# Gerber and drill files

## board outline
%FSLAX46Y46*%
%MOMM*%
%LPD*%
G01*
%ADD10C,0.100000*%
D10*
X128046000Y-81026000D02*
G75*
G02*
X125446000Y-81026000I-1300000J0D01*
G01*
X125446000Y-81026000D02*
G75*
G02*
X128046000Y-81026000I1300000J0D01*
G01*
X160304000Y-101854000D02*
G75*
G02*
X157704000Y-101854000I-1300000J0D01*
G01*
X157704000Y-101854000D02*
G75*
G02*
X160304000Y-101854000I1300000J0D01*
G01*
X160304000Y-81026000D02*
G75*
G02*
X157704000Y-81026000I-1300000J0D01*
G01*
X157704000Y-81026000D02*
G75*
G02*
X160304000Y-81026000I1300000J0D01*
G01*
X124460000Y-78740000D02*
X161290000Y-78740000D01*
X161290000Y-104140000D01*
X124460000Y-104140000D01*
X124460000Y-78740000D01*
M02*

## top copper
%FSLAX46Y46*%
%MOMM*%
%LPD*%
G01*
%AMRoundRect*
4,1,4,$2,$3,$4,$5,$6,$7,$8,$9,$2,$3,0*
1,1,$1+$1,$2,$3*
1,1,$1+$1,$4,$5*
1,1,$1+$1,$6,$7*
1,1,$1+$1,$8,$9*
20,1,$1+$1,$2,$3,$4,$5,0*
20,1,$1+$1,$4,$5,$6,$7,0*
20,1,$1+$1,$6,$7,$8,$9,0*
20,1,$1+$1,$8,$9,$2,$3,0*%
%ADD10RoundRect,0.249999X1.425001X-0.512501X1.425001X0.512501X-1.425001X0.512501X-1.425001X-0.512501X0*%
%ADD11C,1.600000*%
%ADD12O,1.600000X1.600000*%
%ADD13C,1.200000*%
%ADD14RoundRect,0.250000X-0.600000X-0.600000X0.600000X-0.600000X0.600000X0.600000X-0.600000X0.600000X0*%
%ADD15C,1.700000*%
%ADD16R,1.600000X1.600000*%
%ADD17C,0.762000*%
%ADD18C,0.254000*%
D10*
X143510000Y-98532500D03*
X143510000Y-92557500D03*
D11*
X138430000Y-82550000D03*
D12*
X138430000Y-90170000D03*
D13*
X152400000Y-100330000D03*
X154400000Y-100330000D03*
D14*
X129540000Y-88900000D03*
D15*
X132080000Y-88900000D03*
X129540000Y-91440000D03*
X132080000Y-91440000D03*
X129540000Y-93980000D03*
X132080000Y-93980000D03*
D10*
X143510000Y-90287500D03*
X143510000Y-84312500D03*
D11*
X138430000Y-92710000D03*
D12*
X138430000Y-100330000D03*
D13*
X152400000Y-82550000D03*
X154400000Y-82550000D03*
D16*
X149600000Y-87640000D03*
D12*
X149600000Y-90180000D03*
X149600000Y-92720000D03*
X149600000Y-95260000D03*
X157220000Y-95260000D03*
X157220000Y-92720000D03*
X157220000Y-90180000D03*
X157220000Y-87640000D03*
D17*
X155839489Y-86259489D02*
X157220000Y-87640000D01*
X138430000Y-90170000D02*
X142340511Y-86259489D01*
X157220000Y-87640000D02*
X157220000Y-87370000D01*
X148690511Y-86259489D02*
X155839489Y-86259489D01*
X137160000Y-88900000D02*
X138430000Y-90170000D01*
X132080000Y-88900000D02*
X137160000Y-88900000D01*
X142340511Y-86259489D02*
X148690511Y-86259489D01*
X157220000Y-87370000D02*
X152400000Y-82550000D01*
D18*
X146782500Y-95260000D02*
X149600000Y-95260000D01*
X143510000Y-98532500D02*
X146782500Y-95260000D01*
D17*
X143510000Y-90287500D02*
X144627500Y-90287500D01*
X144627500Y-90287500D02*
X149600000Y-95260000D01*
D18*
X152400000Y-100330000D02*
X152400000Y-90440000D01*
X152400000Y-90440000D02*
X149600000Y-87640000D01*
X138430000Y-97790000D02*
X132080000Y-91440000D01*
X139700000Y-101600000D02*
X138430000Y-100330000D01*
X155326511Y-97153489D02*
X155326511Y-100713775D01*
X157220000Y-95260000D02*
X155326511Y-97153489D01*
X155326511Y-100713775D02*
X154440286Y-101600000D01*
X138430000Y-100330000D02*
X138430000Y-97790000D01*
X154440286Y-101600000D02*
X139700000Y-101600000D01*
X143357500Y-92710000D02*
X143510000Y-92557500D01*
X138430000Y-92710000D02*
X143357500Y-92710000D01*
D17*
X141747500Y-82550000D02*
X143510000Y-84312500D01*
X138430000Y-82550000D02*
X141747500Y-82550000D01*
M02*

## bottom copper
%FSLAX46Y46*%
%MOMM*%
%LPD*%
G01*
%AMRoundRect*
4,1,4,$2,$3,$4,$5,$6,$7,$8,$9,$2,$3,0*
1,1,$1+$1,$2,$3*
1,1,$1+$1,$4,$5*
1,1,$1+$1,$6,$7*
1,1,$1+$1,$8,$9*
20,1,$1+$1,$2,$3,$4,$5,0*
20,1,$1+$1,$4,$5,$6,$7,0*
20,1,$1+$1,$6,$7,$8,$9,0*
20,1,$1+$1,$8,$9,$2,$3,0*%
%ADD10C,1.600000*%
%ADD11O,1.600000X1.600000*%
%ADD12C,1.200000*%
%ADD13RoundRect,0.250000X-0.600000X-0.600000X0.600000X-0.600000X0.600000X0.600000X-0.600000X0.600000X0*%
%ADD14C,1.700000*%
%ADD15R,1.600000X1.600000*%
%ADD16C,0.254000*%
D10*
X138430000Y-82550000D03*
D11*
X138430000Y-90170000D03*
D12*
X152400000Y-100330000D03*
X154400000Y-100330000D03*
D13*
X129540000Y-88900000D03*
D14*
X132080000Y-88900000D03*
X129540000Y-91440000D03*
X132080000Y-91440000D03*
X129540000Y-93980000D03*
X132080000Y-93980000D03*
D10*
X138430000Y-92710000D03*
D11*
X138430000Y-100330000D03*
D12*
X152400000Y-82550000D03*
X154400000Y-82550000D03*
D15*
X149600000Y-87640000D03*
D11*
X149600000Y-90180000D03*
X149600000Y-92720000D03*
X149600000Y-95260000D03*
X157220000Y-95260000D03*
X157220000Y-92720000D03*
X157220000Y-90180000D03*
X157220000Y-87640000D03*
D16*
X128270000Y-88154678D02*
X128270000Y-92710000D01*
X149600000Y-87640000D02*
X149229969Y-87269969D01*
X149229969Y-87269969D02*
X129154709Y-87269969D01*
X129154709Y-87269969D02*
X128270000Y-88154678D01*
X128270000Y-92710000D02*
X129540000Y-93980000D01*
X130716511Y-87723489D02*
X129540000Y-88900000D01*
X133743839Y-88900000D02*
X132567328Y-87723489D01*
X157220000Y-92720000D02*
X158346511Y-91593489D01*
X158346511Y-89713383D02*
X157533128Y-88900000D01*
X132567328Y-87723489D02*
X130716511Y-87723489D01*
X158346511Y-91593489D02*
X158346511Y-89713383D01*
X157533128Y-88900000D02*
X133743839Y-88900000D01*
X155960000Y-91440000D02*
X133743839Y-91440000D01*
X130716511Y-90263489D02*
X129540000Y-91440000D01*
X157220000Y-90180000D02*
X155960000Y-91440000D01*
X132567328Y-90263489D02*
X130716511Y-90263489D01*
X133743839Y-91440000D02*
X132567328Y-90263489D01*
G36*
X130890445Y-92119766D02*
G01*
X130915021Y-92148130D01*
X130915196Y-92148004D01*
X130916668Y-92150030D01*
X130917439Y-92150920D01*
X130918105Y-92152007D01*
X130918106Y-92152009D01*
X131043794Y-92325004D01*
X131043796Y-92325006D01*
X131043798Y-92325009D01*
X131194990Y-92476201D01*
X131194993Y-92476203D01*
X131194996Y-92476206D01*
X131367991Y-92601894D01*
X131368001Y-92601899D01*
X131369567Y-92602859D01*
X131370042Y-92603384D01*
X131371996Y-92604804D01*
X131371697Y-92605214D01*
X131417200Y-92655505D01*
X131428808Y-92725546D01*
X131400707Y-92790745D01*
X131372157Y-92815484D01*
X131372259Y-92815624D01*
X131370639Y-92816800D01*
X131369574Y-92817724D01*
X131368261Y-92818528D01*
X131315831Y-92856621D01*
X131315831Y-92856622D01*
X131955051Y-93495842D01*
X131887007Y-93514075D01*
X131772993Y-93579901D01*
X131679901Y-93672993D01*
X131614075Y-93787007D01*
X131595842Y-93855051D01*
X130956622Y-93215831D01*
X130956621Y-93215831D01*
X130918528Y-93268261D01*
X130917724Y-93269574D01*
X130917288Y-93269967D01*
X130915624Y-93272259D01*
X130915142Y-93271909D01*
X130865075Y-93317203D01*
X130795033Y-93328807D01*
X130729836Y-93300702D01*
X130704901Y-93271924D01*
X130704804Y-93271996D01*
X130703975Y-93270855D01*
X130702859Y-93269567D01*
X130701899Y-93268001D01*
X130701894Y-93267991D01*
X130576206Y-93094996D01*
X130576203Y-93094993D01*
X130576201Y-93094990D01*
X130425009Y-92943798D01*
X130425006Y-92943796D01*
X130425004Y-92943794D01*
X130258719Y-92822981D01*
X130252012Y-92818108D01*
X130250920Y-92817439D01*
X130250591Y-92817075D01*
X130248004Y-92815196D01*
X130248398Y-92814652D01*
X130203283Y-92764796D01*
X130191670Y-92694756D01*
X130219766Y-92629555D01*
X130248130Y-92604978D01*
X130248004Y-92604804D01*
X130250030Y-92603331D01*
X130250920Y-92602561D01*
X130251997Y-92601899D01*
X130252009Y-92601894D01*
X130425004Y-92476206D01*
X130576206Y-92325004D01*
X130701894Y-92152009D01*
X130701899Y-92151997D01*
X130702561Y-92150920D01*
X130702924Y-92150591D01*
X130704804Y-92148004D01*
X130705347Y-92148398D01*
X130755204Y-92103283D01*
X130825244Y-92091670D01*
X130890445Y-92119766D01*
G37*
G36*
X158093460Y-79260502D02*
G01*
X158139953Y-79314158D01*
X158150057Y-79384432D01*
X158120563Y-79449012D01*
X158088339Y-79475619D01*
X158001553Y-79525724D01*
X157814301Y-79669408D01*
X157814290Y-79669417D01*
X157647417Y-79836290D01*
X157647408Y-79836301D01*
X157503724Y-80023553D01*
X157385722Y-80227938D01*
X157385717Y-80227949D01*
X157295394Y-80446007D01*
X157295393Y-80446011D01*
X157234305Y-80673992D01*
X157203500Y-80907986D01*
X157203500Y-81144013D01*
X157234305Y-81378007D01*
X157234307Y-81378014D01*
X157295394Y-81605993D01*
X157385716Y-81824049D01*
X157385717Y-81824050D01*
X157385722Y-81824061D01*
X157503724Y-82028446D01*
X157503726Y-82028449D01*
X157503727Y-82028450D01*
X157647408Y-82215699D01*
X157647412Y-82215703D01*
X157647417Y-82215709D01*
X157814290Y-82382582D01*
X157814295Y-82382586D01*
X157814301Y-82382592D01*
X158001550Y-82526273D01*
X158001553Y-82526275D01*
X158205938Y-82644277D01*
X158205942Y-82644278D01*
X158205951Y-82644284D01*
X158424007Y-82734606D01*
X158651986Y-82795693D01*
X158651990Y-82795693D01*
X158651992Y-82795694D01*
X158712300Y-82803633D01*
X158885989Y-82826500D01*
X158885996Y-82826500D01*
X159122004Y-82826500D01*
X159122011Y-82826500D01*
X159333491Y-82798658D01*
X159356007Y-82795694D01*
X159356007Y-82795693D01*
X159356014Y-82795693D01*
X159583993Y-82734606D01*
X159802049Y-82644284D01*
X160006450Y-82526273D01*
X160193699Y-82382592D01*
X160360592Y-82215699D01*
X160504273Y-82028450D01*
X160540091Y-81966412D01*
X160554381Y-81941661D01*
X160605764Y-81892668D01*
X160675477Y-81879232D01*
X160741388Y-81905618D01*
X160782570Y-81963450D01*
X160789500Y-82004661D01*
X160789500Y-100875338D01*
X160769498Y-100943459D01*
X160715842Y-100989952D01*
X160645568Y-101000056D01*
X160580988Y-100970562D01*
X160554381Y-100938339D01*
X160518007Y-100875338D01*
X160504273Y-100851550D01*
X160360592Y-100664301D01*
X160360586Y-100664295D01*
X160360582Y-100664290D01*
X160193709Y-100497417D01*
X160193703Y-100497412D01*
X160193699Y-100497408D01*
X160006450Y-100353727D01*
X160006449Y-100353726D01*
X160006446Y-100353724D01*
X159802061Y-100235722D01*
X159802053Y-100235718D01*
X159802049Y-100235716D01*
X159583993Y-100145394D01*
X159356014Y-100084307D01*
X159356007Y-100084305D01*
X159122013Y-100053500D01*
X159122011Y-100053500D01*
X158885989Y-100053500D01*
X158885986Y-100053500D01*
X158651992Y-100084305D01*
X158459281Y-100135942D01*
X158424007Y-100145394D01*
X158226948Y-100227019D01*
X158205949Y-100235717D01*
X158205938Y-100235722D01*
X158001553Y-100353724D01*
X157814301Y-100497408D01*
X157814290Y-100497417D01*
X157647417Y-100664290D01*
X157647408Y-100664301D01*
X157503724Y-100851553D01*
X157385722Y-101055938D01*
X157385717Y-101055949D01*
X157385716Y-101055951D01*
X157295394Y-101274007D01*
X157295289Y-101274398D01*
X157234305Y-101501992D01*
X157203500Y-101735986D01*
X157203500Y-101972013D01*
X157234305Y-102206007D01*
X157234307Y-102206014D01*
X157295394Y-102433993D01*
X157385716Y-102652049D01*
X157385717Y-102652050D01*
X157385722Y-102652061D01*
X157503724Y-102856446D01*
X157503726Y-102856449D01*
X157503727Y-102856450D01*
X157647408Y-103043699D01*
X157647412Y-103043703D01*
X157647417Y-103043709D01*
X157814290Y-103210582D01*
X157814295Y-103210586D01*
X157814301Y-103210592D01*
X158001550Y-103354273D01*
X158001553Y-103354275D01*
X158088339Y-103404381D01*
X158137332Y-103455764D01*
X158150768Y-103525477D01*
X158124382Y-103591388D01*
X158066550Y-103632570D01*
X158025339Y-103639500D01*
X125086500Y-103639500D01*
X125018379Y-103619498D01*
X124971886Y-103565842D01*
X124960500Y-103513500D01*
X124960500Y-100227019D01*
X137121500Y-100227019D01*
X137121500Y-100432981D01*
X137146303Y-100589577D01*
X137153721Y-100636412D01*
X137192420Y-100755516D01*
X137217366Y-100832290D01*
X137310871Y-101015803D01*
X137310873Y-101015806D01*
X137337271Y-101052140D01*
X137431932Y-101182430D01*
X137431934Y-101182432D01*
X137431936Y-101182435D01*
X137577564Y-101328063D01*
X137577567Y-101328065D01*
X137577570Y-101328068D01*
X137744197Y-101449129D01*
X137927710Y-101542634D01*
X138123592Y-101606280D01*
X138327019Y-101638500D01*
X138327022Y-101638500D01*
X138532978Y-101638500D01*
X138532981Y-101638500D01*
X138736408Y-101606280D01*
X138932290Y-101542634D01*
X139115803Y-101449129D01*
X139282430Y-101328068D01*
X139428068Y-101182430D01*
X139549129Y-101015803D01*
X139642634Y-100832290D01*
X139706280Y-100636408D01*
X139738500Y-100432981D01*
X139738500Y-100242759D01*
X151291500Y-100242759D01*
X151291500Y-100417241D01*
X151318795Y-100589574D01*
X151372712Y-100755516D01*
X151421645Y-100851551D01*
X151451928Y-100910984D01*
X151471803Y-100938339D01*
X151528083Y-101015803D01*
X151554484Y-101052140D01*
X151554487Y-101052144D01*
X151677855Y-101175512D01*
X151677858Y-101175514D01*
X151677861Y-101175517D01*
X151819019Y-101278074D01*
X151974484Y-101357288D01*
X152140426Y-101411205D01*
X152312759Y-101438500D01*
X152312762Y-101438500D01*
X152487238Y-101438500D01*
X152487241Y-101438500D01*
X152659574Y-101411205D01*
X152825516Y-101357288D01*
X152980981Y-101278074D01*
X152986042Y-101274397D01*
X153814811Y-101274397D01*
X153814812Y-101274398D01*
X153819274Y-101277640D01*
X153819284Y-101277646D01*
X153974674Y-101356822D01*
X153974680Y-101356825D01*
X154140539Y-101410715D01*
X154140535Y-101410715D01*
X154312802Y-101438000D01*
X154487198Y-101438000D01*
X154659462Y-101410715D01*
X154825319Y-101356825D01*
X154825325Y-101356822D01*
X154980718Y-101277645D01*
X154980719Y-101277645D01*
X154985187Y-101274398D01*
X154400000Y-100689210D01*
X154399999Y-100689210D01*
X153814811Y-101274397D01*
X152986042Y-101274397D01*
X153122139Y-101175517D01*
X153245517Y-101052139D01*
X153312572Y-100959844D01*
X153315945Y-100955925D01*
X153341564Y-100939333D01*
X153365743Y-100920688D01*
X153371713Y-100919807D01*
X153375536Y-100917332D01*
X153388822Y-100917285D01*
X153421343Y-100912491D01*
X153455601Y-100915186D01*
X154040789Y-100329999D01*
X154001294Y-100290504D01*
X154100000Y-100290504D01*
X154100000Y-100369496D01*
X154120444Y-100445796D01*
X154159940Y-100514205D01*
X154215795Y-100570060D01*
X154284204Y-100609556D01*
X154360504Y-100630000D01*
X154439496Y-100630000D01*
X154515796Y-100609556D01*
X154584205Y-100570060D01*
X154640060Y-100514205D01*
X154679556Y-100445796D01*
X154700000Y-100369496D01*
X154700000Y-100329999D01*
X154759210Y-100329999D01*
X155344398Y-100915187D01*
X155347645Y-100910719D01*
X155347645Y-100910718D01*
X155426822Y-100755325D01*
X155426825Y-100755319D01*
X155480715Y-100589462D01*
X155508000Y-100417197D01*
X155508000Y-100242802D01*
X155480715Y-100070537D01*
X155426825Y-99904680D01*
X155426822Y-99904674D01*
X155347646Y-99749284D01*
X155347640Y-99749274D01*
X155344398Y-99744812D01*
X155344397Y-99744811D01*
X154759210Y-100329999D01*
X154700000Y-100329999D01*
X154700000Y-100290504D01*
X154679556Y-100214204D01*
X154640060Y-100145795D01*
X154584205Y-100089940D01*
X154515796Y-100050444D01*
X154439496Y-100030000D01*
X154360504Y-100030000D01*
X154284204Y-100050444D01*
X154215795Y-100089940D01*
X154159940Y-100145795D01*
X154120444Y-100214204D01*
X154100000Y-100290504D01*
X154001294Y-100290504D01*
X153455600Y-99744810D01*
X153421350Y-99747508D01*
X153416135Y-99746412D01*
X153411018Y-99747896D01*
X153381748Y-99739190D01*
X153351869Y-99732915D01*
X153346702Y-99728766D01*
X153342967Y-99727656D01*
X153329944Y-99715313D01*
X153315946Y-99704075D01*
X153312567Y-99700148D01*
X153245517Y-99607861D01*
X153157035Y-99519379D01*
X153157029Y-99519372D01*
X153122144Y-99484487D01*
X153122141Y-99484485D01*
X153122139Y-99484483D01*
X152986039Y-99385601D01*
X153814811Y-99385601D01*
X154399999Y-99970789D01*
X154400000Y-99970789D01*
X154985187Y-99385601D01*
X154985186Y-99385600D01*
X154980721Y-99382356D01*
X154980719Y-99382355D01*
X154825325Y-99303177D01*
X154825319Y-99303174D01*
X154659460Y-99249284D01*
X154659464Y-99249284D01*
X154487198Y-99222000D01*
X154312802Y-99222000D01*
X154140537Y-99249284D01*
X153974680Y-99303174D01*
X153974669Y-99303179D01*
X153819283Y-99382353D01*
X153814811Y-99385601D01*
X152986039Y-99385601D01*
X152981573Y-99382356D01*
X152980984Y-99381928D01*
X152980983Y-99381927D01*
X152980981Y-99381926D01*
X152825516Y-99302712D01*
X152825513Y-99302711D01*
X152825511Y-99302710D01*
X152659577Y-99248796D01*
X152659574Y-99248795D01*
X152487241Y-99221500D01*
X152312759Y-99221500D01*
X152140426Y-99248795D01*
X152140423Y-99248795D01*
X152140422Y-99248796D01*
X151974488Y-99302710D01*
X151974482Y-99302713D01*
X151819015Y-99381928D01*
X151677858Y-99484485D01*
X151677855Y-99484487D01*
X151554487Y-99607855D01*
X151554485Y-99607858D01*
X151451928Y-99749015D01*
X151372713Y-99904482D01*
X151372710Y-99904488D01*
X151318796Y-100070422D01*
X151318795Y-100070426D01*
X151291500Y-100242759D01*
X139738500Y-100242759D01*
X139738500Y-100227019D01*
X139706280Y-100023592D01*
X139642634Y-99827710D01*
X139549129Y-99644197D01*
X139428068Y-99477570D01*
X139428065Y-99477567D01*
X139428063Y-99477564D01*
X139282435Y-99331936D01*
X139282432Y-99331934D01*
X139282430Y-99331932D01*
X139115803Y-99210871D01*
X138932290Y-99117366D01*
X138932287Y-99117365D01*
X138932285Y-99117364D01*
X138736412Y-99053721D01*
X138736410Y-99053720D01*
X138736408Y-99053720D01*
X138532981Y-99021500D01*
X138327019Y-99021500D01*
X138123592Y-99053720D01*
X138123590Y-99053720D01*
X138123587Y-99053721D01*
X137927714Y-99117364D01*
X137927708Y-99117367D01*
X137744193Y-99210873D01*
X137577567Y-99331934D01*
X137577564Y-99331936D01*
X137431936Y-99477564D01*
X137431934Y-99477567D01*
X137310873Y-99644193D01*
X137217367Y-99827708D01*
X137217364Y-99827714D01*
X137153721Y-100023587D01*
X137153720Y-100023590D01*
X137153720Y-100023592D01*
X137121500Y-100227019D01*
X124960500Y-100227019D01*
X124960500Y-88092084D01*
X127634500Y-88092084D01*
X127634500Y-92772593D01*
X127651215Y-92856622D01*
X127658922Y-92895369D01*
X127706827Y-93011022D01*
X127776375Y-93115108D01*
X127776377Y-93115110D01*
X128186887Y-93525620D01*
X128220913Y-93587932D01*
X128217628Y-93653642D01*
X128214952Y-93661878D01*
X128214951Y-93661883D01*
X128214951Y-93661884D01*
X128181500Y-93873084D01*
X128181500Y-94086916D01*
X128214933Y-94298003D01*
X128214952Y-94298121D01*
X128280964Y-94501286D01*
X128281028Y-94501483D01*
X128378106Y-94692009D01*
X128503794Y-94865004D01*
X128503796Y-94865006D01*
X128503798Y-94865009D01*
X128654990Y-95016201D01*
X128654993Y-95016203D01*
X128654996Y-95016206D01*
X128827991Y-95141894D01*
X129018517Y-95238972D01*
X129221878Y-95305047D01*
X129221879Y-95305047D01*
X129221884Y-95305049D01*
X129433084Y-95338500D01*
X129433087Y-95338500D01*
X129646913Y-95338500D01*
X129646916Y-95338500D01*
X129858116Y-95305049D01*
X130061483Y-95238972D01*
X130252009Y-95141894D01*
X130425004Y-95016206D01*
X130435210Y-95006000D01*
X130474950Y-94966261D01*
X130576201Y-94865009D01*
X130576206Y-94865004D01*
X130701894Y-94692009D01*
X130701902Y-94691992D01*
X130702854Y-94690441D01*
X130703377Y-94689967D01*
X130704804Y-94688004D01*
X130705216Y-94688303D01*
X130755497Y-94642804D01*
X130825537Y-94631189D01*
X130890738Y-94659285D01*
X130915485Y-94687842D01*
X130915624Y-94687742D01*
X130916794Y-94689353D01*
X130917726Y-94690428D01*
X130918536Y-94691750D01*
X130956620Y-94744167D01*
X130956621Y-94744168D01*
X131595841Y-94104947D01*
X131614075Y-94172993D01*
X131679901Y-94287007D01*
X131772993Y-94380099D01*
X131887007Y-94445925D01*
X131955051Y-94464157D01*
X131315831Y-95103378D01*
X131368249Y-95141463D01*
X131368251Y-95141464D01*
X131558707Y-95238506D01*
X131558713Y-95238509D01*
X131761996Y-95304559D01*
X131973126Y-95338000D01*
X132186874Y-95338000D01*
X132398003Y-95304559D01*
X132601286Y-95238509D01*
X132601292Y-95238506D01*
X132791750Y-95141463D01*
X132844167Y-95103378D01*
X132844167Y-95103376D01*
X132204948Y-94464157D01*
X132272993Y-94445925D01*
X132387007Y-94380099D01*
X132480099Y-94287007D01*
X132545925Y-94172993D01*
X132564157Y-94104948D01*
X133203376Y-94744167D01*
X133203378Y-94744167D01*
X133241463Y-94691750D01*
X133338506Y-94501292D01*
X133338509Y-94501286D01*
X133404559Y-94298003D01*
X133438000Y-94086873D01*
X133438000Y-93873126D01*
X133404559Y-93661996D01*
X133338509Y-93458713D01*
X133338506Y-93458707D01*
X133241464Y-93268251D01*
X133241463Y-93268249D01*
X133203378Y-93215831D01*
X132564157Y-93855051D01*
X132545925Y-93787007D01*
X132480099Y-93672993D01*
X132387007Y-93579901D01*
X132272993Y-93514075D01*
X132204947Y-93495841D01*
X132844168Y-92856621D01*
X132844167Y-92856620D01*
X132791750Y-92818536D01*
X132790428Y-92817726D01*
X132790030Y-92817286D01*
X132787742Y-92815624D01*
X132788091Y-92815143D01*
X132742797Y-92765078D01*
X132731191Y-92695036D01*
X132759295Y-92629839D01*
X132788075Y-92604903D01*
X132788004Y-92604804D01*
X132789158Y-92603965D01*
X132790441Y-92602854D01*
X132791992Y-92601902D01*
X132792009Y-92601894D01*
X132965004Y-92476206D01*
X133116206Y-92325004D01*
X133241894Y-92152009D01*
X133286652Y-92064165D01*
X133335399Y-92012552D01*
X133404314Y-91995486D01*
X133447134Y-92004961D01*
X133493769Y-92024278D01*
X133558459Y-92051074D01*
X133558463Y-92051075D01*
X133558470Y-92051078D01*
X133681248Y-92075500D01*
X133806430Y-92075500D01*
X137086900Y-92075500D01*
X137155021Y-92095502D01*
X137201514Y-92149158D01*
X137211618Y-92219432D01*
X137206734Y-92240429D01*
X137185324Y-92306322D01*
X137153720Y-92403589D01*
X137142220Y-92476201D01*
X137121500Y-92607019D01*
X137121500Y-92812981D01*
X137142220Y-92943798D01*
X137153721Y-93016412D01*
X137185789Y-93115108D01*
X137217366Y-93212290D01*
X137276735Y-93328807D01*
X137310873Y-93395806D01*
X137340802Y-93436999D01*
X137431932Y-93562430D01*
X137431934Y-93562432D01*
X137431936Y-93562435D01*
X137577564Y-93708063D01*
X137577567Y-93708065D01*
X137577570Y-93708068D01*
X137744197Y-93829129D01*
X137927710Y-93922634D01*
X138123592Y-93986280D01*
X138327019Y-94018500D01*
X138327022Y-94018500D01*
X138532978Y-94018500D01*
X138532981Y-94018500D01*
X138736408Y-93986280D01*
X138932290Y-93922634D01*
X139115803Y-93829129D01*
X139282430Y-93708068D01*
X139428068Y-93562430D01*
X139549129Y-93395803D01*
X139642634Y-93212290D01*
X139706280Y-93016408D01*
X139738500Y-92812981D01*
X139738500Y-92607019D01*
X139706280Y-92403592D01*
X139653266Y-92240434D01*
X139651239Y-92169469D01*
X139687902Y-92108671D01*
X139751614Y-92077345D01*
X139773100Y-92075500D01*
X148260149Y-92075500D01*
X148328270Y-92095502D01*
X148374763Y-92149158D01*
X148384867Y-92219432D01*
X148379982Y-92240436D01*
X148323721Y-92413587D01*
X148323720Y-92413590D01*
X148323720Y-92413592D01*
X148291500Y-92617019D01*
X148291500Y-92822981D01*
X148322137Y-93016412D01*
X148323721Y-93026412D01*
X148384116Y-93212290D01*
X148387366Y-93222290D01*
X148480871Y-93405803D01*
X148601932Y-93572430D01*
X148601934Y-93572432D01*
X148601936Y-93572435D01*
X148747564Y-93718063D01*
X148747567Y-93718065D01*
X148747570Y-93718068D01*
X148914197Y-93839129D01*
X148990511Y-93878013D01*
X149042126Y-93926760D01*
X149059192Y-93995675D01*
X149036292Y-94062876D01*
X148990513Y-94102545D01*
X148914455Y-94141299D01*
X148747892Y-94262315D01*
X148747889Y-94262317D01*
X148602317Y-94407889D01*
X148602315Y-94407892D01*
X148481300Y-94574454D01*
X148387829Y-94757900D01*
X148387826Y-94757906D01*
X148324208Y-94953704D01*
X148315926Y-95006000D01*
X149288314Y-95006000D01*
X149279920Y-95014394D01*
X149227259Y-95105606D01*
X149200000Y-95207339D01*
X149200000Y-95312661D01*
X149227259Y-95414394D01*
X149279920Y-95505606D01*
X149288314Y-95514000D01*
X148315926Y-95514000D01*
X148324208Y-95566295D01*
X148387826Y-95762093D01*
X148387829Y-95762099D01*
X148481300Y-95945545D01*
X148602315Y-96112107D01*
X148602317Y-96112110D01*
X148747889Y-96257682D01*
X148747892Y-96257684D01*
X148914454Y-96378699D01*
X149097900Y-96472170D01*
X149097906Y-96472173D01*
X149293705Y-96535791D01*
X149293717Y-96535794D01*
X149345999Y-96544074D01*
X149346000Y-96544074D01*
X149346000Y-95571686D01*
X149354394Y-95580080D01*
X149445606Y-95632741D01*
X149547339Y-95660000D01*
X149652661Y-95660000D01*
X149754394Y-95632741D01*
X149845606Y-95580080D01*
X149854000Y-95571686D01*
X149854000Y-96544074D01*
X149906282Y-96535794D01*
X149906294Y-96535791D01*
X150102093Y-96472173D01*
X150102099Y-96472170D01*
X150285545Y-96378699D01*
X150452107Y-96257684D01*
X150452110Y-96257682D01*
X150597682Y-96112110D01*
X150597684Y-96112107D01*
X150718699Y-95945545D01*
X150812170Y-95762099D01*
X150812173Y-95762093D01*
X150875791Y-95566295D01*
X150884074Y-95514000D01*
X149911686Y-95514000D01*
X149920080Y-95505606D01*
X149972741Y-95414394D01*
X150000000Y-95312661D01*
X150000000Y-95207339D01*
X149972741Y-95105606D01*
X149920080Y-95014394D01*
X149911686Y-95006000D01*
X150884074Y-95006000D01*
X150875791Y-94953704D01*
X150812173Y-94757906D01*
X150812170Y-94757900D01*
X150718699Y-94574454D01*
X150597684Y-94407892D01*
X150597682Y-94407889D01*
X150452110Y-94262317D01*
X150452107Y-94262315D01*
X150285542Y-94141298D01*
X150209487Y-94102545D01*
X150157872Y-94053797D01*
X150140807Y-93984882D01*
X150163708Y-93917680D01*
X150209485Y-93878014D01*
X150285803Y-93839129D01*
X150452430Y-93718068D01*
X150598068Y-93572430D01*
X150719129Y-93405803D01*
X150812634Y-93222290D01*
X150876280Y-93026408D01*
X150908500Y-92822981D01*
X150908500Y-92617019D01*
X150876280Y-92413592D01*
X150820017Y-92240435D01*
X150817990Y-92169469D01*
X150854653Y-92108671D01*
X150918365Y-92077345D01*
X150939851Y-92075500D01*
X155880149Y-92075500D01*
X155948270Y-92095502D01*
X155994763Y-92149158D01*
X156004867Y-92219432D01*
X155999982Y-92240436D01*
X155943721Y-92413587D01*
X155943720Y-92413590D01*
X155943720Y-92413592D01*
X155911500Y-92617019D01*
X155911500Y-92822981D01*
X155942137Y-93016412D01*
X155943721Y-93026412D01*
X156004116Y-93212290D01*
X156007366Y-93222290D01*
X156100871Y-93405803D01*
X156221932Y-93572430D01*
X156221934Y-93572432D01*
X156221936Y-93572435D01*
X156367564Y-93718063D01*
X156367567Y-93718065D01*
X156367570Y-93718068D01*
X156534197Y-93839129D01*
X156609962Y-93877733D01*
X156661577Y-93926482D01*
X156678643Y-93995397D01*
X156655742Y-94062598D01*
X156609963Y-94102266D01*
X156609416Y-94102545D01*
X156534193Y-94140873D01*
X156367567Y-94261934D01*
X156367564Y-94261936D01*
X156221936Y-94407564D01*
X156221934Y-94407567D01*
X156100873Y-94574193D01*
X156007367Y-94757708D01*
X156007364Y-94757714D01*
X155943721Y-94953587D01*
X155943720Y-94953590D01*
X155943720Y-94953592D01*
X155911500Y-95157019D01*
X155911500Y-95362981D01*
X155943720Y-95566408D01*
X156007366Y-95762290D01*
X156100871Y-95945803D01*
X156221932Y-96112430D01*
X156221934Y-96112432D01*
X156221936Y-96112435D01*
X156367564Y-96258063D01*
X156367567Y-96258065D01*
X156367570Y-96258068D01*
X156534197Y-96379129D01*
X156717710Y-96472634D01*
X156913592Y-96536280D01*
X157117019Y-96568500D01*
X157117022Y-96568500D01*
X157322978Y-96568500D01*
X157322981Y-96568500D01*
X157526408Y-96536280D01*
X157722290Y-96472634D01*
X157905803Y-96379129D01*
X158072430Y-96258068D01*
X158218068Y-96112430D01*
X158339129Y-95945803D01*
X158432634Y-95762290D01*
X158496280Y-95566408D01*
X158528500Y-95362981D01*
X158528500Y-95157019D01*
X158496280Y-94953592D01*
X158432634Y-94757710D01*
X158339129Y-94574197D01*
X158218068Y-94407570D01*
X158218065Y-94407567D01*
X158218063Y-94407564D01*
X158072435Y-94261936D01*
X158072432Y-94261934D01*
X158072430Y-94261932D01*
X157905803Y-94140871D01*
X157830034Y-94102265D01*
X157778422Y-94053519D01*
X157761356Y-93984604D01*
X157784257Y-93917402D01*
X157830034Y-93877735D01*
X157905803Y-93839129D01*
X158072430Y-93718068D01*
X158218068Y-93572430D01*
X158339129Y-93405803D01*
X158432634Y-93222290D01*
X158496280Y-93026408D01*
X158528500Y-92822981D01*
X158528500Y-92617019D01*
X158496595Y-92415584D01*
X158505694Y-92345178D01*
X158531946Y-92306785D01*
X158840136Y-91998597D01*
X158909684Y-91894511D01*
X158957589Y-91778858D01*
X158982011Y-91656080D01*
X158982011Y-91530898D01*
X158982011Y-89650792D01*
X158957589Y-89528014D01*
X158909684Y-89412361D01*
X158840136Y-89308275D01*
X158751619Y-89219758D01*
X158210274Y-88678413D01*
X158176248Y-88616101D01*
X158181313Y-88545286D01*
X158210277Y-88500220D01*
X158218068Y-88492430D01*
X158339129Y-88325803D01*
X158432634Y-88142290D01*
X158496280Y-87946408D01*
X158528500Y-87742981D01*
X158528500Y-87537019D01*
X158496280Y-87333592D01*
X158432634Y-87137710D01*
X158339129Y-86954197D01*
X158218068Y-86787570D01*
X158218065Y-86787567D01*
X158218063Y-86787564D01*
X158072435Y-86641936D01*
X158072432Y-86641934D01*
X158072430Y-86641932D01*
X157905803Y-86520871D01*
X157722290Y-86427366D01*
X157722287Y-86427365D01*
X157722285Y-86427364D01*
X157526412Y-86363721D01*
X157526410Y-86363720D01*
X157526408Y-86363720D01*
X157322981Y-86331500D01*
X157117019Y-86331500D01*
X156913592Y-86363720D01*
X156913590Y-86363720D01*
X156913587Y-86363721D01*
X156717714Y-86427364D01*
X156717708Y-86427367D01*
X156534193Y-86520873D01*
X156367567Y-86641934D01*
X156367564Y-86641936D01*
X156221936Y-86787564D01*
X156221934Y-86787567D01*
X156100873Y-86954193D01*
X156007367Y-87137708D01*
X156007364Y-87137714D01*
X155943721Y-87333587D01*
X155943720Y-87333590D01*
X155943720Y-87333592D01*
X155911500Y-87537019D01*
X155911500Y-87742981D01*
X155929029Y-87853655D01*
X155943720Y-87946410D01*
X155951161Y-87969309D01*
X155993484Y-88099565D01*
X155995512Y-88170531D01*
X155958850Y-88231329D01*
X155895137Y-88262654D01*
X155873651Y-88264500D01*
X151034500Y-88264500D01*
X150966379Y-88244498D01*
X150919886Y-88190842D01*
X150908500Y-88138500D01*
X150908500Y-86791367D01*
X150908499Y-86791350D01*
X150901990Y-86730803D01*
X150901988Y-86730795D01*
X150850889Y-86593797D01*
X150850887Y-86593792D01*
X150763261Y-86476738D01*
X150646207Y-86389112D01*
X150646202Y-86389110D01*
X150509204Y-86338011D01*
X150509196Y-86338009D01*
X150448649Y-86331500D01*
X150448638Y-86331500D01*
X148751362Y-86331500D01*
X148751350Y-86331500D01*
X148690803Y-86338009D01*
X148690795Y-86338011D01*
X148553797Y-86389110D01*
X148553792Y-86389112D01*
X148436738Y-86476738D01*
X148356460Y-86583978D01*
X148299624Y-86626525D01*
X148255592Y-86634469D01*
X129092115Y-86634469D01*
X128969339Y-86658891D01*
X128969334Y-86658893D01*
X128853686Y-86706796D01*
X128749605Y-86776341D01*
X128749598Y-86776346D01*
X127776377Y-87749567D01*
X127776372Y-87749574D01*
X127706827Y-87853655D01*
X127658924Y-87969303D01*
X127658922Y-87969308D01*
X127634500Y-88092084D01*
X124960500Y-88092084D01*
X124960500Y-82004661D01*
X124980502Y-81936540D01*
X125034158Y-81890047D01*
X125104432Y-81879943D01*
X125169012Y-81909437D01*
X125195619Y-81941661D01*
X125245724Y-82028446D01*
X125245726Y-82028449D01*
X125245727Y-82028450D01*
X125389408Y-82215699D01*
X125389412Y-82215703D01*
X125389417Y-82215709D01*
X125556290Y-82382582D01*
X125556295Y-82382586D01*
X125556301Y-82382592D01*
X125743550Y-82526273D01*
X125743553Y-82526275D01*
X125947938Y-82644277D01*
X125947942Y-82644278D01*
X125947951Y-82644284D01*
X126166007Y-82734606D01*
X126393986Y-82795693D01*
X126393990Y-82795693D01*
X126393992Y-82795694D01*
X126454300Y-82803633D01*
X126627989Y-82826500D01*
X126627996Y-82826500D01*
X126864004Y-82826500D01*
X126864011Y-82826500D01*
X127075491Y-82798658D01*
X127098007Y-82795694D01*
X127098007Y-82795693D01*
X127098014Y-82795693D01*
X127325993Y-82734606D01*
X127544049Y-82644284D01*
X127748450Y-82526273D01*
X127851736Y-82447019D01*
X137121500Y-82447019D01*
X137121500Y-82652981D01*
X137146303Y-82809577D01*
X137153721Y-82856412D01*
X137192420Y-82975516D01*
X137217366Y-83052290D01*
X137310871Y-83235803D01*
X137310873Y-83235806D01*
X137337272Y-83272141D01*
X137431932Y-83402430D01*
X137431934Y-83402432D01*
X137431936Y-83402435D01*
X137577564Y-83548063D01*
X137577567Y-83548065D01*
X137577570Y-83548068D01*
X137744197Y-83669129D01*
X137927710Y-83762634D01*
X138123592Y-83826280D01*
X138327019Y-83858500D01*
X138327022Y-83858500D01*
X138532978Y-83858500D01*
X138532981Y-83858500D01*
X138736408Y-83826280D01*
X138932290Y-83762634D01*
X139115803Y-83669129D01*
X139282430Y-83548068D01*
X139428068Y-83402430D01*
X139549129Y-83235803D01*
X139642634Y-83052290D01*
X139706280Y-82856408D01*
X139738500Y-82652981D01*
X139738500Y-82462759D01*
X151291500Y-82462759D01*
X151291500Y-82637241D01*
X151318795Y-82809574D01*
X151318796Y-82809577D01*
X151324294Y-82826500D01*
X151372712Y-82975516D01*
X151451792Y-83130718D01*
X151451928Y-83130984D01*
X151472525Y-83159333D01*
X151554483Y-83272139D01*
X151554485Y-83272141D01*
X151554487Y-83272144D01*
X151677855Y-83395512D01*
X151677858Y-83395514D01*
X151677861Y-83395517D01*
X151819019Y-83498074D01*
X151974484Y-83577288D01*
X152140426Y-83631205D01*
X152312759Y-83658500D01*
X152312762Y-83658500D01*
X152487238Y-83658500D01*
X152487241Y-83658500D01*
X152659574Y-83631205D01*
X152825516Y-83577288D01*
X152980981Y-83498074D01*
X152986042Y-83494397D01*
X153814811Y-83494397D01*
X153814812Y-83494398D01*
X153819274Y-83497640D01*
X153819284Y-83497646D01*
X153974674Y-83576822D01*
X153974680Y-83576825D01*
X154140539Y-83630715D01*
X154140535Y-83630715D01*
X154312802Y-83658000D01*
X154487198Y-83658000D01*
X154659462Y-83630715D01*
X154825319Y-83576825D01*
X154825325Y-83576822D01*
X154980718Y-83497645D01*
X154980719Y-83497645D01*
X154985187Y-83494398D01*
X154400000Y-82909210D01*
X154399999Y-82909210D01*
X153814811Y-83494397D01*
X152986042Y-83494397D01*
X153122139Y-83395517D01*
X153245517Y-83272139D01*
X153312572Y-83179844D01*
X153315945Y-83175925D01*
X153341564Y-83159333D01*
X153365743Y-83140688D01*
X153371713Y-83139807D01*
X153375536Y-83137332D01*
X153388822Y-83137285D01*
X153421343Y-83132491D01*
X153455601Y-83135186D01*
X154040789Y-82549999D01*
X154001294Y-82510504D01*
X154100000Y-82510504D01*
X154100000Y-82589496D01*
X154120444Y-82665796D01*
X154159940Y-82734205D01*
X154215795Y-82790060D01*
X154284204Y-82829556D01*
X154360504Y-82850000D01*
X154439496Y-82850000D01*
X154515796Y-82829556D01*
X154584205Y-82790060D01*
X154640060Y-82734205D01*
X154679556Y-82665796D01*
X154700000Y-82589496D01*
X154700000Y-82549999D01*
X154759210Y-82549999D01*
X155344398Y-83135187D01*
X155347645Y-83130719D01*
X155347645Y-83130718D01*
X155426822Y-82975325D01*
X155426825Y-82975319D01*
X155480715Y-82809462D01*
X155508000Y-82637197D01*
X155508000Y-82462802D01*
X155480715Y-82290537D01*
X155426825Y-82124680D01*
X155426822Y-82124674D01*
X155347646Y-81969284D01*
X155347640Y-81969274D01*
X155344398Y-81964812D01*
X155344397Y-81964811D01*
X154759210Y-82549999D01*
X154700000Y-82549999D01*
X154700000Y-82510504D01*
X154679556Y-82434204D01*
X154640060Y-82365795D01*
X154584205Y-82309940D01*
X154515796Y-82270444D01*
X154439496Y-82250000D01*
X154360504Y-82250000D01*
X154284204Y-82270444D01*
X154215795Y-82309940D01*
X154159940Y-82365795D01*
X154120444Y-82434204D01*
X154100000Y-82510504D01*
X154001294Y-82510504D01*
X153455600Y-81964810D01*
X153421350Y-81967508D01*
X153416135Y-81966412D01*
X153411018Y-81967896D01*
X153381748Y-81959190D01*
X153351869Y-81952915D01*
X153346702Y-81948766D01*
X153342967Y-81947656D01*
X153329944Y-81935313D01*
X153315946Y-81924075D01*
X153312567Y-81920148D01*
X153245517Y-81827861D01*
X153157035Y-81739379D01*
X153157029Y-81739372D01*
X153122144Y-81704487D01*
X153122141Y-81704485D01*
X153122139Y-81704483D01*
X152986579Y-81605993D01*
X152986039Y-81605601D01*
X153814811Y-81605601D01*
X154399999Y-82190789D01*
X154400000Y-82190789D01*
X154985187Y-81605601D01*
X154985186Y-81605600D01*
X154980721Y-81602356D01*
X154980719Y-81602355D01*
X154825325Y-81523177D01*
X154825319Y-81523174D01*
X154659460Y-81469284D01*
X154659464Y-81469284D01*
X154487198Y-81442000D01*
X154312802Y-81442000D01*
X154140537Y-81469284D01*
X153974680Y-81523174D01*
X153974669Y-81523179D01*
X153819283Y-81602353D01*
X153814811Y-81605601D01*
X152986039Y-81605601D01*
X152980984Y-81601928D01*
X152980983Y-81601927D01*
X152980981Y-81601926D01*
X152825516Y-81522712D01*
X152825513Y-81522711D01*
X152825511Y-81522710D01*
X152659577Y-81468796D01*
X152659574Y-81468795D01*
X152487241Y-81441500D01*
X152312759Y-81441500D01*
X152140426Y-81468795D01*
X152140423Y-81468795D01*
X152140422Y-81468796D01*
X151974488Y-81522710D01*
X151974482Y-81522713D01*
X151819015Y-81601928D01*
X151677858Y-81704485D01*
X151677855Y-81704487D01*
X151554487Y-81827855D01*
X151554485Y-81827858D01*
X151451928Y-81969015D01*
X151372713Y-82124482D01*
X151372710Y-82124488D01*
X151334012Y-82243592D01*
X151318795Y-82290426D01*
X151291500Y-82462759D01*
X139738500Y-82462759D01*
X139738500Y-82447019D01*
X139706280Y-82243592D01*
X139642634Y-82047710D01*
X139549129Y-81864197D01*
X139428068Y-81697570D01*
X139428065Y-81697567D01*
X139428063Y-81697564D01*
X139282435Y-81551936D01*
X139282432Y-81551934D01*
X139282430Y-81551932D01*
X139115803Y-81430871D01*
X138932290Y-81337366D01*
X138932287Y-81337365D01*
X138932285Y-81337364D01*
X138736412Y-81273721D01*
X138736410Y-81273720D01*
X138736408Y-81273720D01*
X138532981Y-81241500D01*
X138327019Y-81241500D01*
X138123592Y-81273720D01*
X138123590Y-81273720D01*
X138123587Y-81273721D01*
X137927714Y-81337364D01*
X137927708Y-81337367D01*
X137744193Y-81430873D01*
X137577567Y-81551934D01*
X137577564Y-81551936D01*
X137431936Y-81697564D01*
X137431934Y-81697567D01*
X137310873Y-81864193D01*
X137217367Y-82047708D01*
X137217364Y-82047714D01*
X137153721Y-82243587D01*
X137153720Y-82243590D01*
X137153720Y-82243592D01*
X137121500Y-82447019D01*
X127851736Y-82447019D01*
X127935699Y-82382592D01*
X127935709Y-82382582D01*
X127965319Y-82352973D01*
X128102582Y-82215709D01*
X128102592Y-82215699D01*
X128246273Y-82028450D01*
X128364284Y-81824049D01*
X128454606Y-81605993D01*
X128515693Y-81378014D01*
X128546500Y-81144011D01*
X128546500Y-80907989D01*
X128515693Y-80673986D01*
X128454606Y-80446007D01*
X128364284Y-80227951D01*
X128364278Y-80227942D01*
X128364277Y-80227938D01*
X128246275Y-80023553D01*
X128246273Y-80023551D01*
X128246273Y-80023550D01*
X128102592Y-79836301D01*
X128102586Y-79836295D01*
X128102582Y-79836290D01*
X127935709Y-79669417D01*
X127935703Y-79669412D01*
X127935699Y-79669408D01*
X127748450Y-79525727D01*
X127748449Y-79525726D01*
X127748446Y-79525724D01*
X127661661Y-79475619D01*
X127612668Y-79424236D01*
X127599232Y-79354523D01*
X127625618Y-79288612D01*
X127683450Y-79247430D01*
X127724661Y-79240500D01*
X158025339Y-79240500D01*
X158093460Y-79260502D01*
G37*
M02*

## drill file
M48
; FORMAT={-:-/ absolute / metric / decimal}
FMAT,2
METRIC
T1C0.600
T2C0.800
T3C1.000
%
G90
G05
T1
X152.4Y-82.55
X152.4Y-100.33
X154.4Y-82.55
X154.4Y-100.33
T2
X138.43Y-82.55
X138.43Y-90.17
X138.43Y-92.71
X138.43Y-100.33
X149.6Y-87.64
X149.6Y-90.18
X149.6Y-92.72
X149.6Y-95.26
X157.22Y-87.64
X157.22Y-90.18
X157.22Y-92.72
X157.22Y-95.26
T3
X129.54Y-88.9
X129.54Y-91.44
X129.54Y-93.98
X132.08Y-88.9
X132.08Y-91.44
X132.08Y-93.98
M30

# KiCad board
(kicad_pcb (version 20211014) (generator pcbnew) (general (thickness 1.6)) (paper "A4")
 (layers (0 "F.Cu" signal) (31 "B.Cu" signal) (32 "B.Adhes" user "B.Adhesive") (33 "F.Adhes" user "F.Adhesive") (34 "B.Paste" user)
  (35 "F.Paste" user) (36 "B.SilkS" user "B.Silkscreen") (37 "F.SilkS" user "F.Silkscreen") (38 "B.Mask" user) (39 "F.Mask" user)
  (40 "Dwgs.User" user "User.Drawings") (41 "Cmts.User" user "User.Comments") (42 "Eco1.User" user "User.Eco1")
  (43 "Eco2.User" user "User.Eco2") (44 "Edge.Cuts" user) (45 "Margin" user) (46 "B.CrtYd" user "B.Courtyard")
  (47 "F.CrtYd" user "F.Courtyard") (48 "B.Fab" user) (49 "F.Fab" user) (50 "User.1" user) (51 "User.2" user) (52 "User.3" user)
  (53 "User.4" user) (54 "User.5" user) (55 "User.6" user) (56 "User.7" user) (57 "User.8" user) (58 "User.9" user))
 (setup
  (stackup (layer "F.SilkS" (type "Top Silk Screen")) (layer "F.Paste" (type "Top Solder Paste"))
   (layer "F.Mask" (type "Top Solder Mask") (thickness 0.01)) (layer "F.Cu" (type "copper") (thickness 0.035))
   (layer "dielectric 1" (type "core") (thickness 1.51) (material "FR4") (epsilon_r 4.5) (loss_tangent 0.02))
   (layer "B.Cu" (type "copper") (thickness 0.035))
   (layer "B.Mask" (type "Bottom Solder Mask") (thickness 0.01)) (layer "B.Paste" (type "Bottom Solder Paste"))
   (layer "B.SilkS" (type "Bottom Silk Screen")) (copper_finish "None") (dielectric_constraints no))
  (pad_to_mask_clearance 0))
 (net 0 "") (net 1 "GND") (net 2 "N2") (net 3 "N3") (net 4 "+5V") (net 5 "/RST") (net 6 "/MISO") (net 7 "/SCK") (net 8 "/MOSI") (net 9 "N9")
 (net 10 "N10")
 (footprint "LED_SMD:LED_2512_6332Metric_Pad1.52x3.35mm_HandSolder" (layer "F.Cu") (at 143.51 95.545 90)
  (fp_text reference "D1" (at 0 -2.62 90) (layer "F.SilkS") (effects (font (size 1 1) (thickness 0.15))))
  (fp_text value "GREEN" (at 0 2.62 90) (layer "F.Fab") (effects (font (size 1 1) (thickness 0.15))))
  (pad "1" smd roundrect (at -2.9875 0 90) (size 1.525 3.35) (layers "F.Cu" "F.Paste" "F.Mask") (roundrect_rratio 0.163934) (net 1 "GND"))
  (pad "2" smd roundrect (at 2.9875 0 90) (size 1.525 3.35) (layers "F.Cu" "F.Paste" "F.Mask") (roundrect_rratio 0.163934) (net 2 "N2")))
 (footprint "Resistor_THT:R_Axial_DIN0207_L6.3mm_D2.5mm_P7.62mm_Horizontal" (layer "F.Cu") (at 138.43 82.55 -90)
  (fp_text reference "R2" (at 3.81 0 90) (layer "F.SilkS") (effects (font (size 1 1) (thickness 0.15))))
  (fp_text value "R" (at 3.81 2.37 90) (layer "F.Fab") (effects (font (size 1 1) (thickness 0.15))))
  (pad "1" thru_hole circle (at 0 0 270) (size 1.6 1.6) (drill 0.8) (layers *.Cu *.Mask) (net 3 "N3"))
  (pad "2" thru_hole oval (at 7.62 0 270) (size 1.6 1.6) (drill 0.8) (layers *.Cu *.Mask) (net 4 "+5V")))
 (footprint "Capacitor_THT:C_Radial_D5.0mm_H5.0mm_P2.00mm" (layer "F.Cu") (at 152.4 100.33)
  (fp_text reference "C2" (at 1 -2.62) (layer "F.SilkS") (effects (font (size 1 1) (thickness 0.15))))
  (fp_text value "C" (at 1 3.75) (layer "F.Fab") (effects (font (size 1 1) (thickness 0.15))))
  (pad "1" thru_hole circle (at 0 0) (size 1.2 1.2) (drill 0.6) (layers *.Cu *.Mask) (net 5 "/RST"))
  (pad "2" thru_hole circle (at 2 0) (size 1.2 1.2) (drill 0.6) (layers *.Cu *.Mask) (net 1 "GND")))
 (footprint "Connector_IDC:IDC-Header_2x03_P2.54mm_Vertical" (layer "F.Cu") (at 129.54 88.9)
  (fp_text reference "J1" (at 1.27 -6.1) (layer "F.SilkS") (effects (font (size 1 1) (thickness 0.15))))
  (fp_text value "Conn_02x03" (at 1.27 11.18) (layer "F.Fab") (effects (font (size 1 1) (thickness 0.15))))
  (pad "1" thru_hole roundrect (at 0 0) (size 1.7 1.7) (drill 1) (layers *.Cu *.Mask) (roundrect_rratio 0.147059) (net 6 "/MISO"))
  (pad "2" thru_hole circle (at 2.54 0) (size 1.7 1.7) (drill 1) (layers *.Cu *.Mask) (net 4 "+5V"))
  (pad "3" thru_hole circle (at 0 2.54) (size 1.7 1.7) (drill 1) (layers *.Cu *.Mask) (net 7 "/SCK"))
  (pad "4" thru_hole circle (at 2.54 2.54) (size 1.7 1.7) (drill 1) (layers *.Cu *.Mask) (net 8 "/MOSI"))
  (pad "5" thru_hole circle (at 0 5.08) (size 1.7 1.7) (drill 1) (layers *.Cu *.Mask) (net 5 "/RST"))
  (pad "6" thru_hole circle (at 2.54 5.08) (size 1.7 1.7) (drill 1) (layers *.Cu *.Mask) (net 1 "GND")))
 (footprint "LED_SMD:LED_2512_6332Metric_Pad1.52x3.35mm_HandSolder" (layer "F.Cu") (at 143.51 87.3 90)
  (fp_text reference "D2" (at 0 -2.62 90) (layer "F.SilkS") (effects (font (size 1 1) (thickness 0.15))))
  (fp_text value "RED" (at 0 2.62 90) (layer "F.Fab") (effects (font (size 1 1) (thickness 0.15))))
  (pad "1" smd roundrect (at -2.9875 0 90) (size 1.525 3.35) (layers "F.Cu" "F.Paste" "F.Mask") (roundrect_rratio 0.163934) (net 1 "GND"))
  (pad "2" smd roundrect (at 2.9875 0 90) (size 1.525 3.35) (layers "F.Cu" "F.Paste" "F.Mask") (roundrect_rratio 0.163934) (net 3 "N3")))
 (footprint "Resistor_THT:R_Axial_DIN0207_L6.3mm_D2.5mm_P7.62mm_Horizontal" (layer "F.Cu") (at 138.43 92.71 -90)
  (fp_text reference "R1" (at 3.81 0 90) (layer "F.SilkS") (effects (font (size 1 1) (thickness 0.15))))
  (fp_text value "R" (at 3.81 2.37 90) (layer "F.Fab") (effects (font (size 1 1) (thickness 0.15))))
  (pad "1" thru_hole circle (at 0 0 270) (size 1.6 1.6) (drill 0.8) (layers *.Cu *.Mask) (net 2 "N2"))
  (pad "2" thru_hole oval (at 7.62 0 270) (size 1.6 1.6) (drill 0.8) (layers *.Cu *.Mask) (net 8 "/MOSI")))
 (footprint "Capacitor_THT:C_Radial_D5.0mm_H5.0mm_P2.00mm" (layer "F.Cu") (at 152.4 82.55)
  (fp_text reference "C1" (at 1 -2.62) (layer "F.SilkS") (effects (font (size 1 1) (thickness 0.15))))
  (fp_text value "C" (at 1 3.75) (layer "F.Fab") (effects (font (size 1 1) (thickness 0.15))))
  (pad "1" thru_hole circle (at 0 0) (size 1.2 1.2) (drill 0.6) (layers *.Cu *.Mask) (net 4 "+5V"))
  (pad "2" thru_hole circle (at 2 0) (size 1.2 1.2) (drill 0.6) (layers *.Cu *.Mask) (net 1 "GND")))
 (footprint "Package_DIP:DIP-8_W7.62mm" (layer "F.Cu") (at 149.6 87.64)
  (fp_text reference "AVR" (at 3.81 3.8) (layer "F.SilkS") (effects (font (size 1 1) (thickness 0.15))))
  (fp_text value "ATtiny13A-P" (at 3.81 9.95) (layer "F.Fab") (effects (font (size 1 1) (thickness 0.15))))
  (pad "1" thru_hole rect (at 0 0) (size 1.6 1.6) (drill 0.8) (layers *.Cu *.Mask) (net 5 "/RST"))
  (pad "2" thru_hole oval (at 0 2.54) (size 1.6 1.6) (drill 0.8) (layers *.Cu *.Mask) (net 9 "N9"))
  (pad "3" thru_hole oval (at 0 5.08) (size 1.6 1.6) (drill 0.8) (layers *.Cu *.Mask) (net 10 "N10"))
  (pad "4" thru_hole oval (at 0 7.62) (size 1.6 1.6) (drill 0.8) (layers *.Cu *.Mask) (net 1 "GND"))
  (pad "5" thru_hole oval (at 7.62 7.62) (size 1.6 1.6) (drill 0.8) (layers *.Cu *.Mask) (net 8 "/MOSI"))
  (pad "6" thru_hole oval (at 7.62 5.08) (size 1.6 1.6) (drill 0.8) (layers *.Cu *.Mask) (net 6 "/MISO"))
  (pad "7" thru_hole oval (at 7.62 2.54) (size 1.6 1.6) (drill 0.8) (layers *.Cu *.Mask) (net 7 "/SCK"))
  (pad "8" thru_hole oval (at 7.62 0) (size 1.6 1.6) (drill 0.8) (layers *.Cu *.Mask) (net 4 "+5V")))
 (gr_circle (center 126.746 81.026) (end 128.046 81.026) (layer "Edge.Cuts") (width 0.1) (fill none))
 (gr_circle (center 159.004 101.854) (end 160.304 101.854) (layer "Edge.Cuts") (width 0.1) (fill none))
 (gr_circle (center 159.004 81.026) (end 160.304 81.026) (layer "Edge.Cuts") (width 0.1) (fill none))
 (gr_rect (start 124.46 78.74) (end 161.29 104.14) (layer "Edge.Cuts") (width 0.1) (fill none))
 (segment (start 155.839489 86.259489) (end 157.22 87.64) (width 0.762) (layer "F.Cu") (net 4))
 (segment (start 138.43 90.17) (end 142.340511 86.259489) (width 0.762) (layer "F.Cu") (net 4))
 (segment (start 157.22 87.64) (end 157.22 87.37) (width 0.762) (layer "F.Cu") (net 4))
 (segment (start 148.690511 86.259489) (end 155.839489 86.259489) (width 0.762) (layer "F.Cu") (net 4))
 (segment (start 137.16 88.9) (end 138.43 90.17) (width 0.762) (layer "F.Cu") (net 4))
 (segment (start 132.08 88.9) (end 137.16 88.9) (width 0.762) (layer "F.Cu") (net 4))
 (segment (start 142.340511 86.259489) (end 148.690511 86.259489) (width 0.762) (layer "F.Cu") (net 4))
 (segment (start 157.22 87.37) (end 152.4 82.55) (width 0.762) (layer "F.Cu") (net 4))
 (segment (start 146.7825 95.26) (end 149.6 95.26) (width 0.254) (layer "F.Cu") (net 1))
 (segment (start 143.51 98.5325) (end 146.7825 95.26) (width 0.254) (layer "F.Cu") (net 1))
 (segment (start 143.51 90.2875) (end 144.6275 90.2875) (width 0.762) (layer "F.Cu") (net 1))
 (segment (start 144.6275 90.2875) (end 149.6 95.26) (width 0.762) (layer "F.Cu") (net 1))
 (segment (start 152.4 100.33) (end 152.4 90.44) (width 0.254) (layer "F.Cu") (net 5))
 (segment (start 152.4 90.44) (end 149.6 87.64) (width 0.254) (layer "F.Cu") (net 5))
 (segment (start 128.27 88.154678) (end 128.27 92.71) (width 0.254) (layer "B.Cu") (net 5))
 (segment (start 149.6 87.64) (end 149.229969 87.269969) (width 0.254) (layer "B.Cu") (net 5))
 (segment (start 149.229969 87.269969) (end 129.154709 87.269969) (width 0.254) (layer "B.Cu") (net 5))
 (segment (start 129.154709 87.269969) (end 128.27 88.154678) (width 0.254) (layer "B.Cu") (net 5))
 (segment (start 128.27 92.71) (end 129.54 93.98) (width 0.254) (layer "B.Cu") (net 5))
 (segment (start 138.43 97.79) (end 132.08 91.44) (width 0.254) (layer "F.Cu") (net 8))
 (segment (start 139.7 101.6) (end 138.43 100.33) (width 0.254) (layer "F.Cu") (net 8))
 (segment (start 155.326511 97.153489) (end 155.326511 100.713775) (width 0.254) (layer "F.Cu") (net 8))
 (segment (start 157.22 95.26) (end 155.326511 97.153489) (width 0.254) (layer "F.Cu") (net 8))
 (segment (start 155.326511 100.713775) (end 154.440286 101.6) (width 0.254) (layer "F.Cu") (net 8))
 (segment (start 138.43 100.33) (end 138.43 97.79) (width 0.254) (layer "F.Cu") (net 8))
 (segment (start 154.440286 101.6) (end 139.7 101.6) (width 0.254) (layer "F.Cu") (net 8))
 (segment (start 130.716511 87.723489) (end 129.54 88.9) (width 0.254) (layer "B.Cu") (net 6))
 (segment (start 133.743839 88.9) (end 132.567328 87.723489) (width 0.254) (layer "B.Cu") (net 6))
 (segment (start 157.22 92.72) (end 158.346511 91.593489) (width 0.254) (layer "B.Cu") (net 6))
 (segment (start 158.346511 89.713383) (end 157.533128 88.9) (width 0.254) (layer "B.Cu") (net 6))
 (segment (start 132.567328 87.723489) (end 130.716511 87.723489) (width 0.254) (layer "B.Cu") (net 6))
 (segment (start 158.346511 91.593489) (end 158.346511 89.713383) (width 0.254) (layer "B.Cu") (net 6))
 (segment (start 157.533128 88.9) (end 133.743839 88.9) (width 0.254) (layer "B.Cu") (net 6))
 (segment (start 155.96 91.44) (end 133.743839 91.44) (width 0.254) (layer "B.Cu") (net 7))
 (segment (start 130.716511 90.263489) (end 129.54 91.44) (width 0.254) (layer "B.Cu") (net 7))
 (segment (start 157.22 90.18) (end 155.96 91.44) (width 0.254) (layer "B.Cu") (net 7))
 (segment (start 132.567328 90.263489) (end 130.716511 90.263489) (width 0.254) (layer "B.Cu") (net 7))
 (segment (start 133.743839 91.44) (end 132.567328 90.263489) (width 0.254) (layer "B.Cu") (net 7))
 (segment (start 143.3575 92.71) (end 143.51 92.5575) (width 0.254) (layer "F.Cu") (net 2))
 (segment (start 138.43 92.71) (end 143.3575 92.71) (width 0.254) (layer "F.Cu") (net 2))
 (segment (start 141.7475 82.55) (end 143.51 84.3125) (width 0.762) (layer "F.Cu") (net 3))
 (segment (start 138.43 82.55) (end 141.7475 82.55) (width 0.762) (layer "F.Cu") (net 3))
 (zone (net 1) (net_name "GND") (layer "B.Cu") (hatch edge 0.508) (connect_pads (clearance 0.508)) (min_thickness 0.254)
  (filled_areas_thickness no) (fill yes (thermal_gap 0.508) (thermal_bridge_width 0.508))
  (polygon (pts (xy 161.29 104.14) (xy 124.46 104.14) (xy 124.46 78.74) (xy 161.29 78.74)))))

